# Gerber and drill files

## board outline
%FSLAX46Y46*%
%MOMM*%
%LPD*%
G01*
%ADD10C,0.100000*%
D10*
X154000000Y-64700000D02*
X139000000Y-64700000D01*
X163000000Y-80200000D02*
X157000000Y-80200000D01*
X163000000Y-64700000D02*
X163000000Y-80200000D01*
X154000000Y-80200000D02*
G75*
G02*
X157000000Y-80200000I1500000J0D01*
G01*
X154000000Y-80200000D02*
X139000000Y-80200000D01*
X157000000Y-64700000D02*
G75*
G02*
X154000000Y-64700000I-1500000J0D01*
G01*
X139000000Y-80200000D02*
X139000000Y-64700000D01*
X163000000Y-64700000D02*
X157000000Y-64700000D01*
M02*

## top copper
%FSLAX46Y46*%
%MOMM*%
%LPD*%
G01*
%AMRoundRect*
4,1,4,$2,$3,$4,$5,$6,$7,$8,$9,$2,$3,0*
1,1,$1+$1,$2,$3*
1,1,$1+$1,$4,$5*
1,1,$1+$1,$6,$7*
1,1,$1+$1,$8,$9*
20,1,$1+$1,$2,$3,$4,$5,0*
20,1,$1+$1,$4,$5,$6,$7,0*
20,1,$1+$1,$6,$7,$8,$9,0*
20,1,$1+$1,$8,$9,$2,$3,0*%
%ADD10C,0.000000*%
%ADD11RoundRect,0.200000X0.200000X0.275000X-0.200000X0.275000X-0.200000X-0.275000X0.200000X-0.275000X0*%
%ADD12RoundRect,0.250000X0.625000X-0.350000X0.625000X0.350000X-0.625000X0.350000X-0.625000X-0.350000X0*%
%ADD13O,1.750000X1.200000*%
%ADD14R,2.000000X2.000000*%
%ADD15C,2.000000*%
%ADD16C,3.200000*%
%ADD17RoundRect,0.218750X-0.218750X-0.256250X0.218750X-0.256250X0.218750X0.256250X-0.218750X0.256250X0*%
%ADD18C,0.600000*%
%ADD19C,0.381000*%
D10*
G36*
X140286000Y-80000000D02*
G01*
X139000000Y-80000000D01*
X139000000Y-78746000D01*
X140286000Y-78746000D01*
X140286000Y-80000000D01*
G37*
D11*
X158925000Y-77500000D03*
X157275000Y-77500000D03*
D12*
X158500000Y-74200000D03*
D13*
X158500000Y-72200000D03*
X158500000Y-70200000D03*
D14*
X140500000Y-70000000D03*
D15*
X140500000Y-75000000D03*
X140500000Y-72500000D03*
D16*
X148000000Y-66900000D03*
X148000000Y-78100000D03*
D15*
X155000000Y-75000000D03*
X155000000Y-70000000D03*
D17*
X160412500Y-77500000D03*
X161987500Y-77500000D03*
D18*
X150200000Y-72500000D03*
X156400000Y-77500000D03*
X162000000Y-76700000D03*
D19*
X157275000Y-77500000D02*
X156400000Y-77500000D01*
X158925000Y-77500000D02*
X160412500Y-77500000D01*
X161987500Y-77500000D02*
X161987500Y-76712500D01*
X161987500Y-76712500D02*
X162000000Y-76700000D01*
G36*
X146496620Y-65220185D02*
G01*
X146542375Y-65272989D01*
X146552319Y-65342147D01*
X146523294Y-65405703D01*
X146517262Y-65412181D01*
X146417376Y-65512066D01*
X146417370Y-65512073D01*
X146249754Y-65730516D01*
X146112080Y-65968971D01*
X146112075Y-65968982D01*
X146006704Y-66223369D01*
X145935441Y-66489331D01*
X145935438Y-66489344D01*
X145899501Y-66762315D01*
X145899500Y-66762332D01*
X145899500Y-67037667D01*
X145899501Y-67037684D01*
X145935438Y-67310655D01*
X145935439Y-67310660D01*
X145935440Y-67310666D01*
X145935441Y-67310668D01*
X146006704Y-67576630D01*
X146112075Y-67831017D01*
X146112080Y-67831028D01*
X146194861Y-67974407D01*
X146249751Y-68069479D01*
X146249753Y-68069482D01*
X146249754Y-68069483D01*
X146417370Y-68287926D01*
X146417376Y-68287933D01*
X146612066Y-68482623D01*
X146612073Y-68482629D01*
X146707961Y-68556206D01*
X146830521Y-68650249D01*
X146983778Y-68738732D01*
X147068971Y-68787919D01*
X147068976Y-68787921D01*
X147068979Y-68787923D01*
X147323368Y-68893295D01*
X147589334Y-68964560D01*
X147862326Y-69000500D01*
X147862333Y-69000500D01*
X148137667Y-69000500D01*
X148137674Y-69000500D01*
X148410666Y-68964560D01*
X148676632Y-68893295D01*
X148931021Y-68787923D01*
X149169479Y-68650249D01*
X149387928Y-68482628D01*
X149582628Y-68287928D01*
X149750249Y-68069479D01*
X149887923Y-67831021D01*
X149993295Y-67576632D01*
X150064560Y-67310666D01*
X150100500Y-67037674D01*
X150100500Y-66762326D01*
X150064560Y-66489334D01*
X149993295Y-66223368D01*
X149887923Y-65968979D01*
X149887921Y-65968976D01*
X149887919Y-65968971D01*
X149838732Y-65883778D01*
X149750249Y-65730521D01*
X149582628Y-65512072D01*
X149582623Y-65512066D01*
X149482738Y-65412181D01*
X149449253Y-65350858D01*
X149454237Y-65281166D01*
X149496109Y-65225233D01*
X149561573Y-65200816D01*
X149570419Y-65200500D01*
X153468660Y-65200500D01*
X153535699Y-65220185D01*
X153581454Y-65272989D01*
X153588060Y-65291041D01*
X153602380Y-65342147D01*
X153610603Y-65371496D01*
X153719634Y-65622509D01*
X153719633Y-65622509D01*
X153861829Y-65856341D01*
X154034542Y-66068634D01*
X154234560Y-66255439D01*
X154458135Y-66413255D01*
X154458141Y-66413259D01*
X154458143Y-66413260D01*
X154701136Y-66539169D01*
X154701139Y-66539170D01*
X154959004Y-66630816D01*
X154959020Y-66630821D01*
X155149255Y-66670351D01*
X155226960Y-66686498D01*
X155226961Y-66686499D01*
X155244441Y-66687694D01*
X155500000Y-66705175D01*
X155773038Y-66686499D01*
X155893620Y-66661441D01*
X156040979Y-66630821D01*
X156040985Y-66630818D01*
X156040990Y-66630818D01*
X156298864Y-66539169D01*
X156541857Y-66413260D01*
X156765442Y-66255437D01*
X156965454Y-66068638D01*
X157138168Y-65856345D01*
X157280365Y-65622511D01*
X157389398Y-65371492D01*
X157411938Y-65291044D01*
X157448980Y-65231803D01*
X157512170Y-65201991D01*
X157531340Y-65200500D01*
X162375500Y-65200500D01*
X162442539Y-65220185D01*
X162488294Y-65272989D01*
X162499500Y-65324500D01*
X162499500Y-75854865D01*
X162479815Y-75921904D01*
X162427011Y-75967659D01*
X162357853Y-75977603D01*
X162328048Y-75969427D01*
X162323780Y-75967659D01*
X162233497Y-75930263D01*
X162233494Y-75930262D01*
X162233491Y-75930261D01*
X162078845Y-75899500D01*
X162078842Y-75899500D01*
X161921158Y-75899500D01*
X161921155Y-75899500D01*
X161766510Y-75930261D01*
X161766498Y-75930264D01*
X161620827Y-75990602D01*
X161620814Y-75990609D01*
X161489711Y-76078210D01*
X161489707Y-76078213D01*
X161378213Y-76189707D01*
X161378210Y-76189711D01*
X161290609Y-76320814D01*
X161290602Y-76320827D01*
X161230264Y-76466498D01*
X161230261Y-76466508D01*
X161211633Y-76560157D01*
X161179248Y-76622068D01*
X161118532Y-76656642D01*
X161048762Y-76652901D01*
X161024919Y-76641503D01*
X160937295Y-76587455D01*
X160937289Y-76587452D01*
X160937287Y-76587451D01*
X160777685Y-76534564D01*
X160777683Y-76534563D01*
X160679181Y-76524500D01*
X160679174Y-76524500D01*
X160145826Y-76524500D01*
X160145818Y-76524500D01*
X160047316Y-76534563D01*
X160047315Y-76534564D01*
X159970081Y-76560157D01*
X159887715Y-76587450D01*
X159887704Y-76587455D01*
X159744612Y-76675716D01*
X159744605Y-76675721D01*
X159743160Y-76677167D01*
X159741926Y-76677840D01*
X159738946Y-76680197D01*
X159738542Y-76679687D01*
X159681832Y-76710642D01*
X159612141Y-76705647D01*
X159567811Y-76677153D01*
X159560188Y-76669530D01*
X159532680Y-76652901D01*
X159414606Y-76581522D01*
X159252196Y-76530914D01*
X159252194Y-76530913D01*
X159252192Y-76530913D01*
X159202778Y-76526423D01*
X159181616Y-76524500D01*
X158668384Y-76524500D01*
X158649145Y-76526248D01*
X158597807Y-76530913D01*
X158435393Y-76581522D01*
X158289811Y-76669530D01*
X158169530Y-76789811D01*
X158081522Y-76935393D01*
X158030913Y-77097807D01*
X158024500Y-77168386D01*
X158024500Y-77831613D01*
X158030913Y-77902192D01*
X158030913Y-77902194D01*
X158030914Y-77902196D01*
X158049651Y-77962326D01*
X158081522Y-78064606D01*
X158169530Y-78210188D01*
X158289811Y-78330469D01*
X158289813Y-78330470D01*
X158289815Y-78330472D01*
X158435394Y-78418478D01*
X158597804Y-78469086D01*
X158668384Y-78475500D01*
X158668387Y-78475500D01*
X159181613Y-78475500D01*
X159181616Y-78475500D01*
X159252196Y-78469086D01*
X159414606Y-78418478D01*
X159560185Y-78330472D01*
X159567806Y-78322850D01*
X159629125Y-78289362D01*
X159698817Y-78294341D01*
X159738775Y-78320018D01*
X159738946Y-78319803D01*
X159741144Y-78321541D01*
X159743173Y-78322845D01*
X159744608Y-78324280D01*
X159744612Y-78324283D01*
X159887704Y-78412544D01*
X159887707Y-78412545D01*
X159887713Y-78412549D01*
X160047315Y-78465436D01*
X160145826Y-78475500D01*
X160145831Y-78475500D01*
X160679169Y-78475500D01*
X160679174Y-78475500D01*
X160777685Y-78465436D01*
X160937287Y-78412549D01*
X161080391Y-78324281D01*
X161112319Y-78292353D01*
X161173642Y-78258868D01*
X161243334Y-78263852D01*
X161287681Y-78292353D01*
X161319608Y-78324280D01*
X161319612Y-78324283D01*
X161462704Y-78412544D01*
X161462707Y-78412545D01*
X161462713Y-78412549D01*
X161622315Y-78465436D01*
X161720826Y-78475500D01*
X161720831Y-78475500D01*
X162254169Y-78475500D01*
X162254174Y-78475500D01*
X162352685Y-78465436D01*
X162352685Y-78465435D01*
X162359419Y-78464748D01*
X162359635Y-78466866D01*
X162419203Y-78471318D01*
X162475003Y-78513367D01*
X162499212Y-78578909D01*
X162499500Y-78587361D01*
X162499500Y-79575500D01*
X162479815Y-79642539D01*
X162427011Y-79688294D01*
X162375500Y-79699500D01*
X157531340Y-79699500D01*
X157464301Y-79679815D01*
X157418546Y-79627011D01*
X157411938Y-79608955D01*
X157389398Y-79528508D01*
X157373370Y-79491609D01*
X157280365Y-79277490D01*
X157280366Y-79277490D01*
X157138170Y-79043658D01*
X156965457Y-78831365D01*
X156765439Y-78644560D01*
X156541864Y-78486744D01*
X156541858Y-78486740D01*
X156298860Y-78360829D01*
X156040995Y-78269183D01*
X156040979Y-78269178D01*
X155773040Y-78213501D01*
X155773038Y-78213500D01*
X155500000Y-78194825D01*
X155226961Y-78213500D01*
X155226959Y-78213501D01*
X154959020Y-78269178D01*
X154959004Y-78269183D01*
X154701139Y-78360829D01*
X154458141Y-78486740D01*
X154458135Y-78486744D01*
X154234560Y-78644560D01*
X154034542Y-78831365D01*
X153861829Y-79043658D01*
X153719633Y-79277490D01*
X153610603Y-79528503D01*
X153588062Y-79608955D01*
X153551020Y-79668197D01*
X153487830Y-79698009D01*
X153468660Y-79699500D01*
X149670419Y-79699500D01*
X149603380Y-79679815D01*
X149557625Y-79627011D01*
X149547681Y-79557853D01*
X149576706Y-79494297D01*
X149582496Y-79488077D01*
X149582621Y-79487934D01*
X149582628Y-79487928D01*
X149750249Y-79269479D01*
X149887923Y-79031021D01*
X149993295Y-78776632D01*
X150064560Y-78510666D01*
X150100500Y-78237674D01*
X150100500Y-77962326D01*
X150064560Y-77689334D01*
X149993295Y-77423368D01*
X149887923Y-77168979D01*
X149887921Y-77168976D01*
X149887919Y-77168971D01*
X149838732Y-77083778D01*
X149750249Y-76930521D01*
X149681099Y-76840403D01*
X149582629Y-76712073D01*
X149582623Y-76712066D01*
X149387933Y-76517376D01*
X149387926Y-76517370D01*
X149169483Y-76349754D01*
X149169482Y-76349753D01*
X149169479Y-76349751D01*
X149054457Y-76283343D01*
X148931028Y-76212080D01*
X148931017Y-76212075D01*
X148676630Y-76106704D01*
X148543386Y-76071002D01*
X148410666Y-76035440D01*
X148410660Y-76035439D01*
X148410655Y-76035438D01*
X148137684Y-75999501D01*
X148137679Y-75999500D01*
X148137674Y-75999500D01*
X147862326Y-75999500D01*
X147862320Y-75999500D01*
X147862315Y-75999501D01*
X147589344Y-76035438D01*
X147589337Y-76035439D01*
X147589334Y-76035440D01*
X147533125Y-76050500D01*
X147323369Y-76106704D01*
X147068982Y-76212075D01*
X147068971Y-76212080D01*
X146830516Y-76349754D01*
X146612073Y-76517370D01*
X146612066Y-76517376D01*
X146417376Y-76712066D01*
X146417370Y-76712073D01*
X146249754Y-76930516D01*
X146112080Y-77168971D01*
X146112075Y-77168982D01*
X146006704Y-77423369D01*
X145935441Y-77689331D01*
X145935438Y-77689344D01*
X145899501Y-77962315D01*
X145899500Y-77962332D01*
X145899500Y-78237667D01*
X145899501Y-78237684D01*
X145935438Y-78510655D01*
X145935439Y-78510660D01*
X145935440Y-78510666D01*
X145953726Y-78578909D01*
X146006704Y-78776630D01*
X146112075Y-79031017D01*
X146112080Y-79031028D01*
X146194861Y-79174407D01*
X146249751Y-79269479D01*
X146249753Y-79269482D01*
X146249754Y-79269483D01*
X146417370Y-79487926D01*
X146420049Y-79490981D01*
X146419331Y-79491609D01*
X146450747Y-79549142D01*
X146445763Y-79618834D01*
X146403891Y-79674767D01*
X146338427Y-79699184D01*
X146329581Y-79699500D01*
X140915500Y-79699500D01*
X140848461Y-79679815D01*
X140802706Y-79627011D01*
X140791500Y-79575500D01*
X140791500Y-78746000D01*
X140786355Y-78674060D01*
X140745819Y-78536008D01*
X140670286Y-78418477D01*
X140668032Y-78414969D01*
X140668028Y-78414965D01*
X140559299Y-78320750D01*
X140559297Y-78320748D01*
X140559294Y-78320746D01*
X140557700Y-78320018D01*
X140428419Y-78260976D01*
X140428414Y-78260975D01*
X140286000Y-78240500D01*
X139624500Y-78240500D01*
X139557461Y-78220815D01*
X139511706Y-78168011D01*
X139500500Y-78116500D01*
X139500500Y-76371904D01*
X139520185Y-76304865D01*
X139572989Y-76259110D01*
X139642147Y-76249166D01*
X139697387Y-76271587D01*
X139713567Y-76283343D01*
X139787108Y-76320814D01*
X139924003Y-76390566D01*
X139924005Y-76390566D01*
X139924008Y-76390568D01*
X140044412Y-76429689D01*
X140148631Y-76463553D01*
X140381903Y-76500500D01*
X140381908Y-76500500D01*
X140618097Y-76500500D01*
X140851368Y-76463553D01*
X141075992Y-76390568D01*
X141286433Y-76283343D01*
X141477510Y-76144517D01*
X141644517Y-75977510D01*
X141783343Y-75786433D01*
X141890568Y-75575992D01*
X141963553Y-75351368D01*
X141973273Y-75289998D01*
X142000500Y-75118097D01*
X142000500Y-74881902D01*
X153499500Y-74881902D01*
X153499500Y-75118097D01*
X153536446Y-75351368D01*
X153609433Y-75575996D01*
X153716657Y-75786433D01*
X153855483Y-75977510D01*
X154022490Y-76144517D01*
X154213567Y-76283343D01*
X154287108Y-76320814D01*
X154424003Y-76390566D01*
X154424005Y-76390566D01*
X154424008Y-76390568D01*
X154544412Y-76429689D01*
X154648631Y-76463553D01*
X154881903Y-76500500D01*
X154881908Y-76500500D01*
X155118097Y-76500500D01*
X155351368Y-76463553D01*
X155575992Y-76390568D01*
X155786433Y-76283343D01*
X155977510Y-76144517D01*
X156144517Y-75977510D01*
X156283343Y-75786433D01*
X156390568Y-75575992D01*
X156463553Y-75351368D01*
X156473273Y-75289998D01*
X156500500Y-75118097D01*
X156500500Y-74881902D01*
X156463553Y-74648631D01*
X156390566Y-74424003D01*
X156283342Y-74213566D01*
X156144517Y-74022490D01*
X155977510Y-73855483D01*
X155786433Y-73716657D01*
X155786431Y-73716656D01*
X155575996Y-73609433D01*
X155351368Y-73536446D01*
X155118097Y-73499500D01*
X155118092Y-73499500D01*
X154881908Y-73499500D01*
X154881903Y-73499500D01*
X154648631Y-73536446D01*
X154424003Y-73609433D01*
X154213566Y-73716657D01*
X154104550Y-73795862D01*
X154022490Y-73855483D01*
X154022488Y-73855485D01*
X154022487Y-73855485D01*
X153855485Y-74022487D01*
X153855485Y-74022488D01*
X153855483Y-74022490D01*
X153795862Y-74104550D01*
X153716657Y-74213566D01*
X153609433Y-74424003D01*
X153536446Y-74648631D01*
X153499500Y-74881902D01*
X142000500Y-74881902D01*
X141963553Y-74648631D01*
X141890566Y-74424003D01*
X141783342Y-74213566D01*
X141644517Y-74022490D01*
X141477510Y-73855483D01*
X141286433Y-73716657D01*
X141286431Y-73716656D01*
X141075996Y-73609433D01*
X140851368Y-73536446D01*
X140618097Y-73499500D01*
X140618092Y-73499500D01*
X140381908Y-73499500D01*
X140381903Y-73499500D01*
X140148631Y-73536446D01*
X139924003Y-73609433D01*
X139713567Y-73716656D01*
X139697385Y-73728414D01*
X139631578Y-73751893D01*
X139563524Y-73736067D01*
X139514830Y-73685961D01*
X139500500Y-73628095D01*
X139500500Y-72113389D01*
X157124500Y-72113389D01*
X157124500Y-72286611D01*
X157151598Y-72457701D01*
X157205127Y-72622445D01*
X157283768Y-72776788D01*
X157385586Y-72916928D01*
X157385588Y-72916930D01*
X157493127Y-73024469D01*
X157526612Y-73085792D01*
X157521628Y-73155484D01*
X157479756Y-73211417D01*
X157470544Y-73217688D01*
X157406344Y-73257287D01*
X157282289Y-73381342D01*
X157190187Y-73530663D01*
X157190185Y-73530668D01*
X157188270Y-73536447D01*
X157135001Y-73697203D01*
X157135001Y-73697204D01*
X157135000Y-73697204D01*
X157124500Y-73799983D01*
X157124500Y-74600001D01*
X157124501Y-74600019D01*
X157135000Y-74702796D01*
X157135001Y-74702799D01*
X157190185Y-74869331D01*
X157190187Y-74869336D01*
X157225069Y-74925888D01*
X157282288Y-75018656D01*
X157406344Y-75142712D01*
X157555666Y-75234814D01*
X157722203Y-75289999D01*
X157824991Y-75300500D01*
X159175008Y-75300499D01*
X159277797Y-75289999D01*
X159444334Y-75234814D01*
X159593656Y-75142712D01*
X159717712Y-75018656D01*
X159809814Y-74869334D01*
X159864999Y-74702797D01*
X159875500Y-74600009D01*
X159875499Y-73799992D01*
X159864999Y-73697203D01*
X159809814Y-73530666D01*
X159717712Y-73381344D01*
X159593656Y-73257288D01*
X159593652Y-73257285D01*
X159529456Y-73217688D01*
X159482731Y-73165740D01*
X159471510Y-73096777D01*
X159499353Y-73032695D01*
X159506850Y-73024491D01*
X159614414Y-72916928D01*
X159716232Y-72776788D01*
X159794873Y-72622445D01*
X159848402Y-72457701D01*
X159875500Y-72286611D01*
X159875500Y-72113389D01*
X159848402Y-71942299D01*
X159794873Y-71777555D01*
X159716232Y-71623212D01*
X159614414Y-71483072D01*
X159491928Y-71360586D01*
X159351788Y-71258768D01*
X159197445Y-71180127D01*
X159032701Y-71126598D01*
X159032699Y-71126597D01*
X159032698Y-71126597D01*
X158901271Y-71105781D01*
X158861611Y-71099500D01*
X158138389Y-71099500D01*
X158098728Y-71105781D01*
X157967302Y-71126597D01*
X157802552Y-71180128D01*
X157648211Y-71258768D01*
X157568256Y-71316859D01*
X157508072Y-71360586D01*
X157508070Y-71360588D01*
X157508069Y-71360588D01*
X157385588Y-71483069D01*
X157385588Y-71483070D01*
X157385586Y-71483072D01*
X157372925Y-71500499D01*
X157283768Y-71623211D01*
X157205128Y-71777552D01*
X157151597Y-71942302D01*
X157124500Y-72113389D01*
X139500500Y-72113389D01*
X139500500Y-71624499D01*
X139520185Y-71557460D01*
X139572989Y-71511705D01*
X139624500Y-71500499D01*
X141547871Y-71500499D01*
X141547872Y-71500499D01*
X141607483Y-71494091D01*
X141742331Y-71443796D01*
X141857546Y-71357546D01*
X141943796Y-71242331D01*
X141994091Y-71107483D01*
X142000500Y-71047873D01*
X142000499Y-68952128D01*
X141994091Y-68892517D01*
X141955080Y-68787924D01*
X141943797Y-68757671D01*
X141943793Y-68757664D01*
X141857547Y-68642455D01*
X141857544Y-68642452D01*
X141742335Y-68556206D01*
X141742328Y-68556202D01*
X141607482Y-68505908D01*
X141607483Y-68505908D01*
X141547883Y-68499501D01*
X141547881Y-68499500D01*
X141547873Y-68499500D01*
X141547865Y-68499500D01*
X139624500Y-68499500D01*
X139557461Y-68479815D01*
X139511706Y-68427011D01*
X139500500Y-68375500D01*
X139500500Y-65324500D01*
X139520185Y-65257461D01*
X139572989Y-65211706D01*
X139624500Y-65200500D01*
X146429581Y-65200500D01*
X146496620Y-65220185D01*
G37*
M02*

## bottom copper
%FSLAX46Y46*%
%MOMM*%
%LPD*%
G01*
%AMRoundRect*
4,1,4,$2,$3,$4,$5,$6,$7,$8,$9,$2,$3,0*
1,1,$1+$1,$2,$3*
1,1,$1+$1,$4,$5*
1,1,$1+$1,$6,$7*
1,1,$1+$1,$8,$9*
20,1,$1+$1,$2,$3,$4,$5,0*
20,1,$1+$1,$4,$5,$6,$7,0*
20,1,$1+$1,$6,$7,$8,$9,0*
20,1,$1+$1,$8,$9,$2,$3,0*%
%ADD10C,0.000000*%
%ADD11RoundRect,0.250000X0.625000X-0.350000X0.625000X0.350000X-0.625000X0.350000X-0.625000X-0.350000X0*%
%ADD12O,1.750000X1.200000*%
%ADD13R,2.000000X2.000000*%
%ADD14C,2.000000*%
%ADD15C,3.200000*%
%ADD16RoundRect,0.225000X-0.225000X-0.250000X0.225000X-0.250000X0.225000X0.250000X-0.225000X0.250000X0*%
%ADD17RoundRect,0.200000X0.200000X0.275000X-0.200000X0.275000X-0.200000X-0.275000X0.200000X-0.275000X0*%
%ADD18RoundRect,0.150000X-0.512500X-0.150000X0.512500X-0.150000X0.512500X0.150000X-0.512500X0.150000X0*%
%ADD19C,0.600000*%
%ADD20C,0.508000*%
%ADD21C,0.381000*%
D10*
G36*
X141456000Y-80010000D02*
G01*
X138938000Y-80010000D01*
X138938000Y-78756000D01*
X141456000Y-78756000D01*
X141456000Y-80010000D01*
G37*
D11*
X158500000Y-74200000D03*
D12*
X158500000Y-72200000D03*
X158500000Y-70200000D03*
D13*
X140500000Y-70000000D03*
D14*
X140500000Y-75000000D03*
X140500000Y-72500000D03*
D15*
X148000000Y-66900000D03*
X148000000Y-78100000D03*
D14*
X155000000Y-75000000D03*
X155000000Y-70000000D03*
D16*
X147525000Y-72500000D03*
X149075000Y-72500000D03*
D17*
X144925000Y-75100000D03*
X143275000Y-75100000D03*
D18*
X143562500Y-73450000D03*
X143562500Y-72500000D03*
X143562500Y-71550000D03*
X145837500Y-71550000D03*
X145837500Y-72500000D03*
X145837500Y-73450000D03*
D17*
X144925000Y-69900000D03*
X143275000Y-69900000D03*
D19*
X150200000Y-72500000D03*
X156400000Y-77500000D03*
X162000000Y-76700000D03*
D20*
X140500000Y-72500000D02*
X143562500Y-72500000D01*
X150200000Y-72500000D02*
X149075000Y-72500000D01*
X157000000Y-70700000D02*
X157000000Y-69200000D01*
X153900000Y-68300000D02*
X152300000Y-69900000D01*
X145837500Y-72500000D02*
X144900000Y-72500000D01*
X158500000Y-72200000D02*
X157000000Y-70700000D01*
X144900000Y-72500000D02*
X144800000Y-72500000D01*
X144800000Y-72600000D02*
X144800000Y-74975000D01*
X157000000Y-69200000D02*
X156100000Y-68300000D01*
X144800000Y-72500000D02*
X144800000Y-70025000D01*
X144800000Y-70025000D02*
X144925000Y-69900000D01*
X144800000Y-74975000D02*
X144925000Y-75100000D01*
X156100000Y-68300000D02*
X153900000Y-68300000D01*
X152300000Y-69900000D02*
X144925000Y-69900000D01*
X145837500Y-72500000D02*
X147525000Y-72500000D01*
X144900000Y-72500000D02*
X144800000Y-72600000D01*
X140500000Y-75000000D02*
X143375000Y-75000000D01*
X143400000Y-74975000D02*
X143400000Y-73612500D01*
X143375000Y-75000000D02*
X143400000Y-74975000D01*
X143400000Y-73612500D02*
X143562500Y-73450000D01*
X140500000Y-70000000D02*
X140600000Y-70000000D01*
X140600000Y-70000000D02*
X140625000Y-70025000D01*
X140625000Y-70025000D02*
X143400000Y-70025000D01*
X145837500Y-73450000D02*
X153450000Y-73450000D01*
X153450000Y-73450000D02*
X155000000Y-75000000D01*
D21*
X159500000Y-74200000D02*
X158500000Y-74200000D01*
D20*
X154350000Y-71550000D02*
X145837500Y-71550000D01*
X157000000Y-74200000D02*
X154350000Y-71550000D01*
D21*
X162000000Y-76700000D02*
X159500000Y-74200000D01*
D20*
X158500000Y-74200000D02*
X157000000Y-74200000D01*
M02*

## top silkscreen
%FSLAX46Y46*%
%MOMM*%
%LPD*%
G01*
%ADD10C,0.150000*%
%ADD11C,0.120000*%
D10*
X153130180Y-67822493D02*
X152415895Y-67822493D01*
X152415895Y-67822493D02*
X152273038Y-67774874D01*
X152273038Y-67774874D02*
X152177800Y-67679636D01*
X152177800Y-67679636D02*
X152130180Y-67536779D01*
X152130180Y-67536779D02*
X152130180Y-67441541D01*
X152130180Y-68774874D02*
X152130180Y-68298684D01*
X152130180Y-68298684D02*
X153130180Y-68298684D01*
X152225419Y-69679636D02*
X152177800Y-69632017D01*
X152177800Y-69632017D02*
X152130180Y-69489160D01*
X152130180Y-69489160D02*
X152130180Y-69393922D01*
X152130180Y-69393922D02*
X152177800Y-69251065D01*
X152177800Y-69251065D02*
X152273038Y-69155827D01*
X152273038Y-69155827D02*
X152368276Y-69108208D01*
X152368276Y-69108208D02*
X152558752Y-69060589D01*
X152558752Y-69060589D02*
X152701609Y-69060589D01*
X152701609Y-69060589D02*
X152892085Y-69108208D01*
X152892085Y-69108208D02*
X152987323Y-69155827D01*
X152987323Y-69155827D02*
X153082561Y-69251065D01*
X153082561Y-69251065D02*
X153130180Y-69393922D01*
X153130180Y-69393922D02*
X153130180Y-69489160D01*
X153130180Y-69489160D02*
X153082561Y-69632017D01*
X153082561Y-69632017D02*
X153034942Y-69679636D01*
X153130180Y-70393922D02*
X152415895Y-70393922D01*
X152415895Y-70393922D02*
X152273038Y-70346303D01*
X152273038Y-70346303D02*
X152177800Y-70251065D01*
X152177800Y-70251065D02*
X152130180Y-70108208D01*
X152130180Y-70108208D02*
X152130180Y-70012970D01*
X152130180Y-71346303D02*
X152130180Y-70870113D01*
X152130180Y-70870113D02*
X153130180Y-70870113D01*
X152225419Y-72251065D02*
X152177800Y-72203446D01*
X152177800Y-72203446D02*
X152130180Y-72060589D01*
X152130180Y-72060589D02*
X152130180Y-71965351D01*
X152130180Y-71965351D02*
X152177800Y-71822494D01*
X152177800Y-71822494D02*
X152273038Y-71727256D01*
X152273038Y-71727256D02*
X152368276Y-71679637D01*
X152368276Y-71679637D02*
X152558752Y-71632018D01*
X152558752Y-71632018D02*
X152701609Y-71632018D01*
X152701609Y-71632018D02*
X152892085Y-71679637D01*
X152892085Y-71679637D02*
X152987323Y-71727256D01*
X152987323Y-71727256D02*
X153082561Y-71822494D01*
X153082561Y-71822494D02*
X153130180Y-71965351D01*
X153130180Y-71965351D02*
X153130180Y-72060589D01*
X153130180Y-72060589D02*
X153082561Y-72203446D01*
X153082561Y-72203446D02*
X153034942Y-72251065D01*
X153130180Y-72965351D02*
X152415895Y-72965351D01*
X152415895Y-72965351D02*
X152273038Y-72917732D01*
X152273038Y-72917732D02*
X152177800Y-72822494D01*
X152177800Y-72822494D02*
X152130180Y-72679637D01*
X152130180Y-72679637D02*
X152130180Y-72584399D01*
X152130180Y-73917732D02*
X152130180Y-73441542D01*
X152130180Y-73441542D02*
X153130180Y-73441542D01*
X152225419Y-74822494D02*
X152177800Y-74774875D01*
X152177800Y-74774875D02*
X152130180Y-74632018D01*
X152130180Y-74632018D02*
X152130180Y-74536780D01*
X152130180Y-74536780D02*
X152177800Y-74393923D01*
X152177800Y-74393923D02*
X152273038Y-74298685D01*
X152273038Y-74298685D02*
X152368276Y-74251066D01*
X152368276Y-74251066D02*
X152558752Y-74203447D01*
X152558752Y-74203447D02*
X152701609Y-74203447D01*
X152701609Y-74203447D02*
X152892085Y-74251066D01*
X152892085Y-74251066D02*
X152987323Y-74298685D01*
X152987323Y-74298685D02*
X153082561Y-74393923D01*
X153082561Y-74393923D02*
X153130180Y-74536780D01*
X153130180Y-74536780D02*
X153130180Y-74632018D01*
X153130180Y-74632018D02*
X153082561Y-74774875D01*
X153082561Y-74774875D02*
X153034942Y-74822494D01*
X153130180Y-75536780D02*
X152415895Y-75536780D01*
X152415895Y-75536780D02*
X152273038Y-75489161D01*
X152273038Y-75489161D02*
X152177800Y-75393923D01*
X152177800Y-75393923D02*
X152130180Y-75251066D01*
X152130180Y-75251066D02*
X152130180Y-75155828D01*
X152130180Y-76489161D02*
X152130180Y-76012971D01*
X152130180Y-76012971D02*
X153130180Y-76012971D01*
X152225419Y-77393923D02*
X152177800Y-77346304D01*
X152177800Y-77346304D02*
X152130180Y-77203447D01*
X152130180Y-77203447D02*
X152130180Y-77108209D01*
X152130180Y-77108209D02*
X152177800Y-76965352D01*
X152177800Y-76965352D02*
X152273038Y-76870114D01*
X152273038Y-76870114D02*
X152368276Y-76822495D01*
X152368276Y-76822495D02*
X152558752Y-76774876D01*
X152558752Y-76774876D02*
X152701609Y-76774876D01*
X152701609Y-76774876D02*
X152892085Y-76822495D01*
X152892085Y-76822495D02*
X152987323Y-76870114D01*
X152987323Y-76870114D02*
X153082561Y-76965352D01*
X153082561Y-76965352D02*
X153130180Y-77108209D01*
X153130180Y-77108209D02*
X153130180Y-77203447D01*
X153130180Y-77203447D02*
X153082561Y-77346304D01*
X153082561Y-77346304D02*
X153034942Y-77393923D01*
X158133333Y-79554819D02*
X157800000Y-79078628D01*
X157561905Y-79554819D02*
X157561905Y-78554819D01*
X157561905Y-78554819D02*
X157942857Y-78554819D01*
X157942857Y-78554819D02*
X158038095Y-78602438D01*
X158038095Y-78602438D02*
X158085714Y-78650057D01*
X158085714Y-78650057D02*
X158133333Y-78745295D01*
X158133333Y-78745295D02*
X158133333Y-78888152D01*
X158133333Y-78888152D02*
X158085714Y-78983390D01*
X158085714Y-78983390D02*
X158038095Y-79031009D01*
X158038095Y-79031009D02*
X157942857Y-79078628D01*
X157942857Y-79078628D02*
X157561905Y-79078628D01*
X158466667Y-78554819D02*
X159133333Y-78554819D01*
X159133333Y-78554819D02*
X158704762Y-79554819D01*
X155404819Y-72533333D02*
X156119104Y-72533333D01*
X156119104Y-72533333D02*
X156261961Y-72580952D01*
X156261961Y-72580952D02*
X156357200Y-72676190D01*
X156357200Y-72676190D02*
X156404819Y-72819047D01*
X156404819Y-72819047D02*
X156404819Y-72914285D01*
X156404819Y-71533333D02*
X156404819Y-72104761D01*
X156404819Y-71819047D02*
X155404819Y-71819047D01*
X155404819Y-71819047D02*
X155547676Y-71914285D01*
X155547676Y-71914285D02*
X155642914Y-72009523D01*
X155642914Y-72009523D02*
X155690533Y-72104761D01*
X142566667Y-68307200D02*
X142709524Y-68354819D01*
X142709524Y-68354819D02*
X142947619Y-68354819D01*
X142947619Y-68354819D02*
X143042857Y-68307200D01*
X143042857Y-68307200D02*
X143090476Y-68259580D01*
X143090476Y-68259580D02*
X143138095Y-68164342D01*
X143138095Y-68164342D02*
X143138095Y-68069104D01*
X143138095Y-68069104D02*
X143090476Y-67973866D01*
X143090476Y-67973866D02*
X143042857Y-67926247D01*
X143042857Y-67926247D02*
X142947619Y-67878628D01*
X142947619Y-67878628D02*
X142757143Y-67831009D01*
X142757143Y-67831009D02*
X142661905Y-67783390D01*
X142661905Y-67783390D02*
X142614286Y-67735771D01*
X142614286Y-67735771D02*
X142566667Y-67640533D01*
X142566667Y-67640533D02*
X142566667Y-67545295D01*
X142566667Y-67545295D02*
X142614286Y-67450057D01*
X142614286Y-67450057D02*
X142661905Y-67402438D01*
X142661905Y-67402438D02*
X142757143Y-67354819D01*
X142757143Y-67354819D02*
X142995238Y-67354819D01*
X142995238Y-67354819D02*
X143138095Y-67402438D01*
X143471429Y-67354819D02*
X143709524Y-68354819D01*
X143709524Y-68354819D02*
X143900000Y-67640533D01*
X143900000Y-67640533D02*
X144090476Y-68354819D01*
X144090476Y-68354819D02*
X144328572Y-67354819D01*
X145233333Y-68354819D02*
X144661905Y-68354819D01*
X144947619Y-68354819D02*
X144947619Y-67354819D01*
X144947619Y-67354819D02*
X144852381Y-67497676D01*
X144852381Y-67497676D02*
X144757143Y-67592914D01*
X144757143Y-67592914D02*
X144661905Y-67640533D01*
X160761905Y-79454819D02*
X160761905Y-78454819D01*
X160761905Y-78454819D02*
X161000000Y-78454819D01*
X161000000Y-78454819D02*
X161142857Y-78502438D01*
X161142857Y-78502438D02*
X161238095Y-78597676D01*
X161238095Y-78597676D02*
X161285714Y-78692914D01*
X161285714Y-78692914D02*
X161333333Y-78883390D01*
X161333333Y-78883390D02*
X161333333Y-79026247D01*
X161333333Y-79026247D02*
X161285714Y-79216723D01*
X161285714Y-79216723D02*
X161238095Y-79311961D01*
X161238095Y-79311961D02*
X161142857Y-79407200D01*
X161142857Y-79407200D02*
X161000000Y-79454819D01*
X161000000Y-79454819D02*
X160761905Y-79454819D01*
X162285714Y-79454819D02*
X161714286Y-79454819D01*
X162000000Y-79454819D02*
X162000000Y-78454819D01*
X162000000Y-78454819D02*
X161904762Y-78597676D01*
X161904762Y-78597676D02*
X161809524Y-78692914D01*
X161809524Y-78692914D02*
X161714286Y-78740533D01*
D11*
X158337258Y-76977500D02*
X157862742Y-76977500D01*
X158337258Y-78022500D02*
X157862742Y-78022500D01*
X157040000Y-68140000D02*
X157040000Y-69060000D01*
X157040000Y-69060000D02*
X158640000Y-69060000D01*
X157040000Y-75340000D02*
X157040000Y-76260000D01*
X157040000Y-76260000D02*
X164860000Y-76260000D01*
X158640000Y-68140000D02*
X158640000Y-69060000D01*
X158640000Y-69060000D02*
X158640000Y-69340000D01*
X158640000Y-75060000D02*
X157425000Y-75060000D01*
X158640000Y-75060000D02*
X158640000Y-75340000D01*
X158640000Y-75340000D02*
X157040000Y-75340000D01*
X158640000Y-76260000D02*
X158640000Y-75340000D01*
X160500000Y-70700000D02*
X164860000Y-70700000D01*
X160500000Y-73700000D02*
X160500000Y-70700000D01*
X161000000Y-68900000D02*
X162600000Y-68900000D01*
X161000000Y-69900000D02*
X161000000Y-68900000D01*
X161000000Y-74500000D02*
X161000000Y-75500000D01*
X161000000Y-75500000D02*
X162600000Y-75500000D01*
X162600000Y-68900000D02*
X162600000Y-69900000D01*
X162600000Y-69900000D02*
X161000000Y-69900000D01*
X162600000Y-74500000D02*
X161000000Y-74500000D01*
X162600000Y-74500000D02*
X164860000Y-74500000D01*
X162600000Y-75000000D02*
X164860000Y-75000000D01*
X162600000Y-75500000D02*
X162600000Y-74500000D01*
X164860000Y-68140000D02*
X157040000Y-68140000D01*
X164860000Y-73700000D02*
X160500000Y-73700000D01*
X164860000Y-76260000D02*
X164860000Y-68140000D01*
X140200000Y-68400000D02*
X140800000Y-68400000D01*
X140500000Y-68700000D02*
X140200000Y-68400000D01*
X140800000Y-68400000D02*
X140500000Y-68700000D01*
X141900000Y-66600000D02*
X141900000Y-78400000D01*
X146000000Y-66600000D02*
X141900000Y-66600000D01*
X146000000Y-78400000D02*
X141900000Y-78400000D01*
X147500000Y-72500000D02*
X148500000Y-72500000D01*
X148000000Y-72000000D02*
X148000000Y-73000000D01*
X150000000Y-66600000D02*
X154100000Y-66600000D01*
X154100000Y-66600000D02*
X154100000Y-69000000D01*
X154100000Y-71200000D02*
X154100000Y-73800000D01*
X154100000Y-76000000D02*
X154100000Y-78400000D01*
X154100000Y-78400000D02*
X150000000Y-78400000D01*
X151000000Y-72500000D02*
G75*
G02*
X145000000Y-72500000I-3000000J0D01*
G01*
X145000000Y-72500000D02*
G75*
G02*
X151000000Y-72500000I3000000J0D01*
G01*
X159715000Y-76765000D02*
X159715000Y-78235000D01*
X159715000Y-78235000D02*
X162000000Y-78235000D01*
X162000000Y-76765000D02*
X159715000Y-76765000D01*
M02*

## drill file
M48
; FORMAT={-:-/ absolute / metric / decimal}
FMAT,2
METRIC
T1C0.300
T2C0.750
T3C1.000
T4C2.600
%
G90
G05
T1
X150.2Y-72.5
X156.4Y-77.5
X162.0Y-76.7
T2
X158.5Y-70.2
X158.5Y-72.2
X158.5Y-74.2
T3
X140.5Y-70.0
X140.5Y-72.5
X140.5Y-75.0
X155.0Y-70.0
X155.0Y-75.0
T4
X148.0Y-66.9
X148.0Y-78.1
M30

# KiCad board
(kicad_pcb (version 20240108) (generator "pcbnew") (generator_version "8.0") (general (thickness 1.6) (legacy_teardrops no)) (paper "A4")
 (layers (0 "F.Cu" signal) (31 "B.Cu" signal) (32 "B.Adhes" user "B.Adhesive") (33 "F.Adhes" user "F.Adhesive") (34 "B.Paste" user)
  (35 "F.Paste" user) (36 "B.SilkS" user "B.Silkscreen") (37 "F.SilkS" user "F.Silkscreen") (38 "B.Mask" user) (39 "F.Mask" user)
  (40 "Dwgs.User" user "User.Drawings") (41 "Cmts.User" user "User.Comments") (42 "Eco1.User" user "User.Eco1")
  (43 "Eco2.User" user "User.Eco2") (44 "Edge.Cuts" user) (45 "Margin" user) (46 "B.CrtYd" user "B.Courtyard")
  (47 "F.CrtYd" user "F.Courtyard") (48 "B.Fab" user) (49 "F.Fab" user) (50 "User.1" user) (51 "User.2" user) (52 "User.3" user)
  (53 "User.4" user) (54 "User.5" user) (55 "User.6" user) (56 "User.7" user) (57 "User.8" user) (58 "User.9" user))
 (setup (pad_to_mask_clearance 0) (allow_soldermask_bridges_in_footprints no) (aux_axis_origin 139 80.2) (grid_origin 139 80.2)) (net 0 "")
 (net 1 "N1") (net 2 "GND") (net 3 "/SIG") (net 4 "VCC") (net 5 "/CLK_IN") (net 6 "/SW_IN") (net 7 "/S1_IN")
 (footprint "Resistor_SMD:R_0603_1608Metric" (layer "F.Cu") (at 158.1 77.5 180)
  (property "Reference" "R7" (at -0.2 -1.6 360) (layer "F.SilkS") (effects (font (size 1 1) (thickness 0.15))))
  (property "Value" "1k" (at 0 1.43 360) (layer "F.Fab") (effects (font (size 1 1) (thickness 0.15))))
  (fp_line (start -0.237258 0.5225) (end 0.237258 0.5225) (stroke (width 0.12) (type solid)) (layer "F.SilkS"))
  (fp_line (start -0.237258 -0.5225) (end 0.237258 -0.5225) (stroke (width 0.12) (type solid)) (layer "F.SilkS"))
  (pad "1" smd roundrect (at -0.825 0 180) (size 0.8 0.95) (layers "F.Cu" "F.Paste" "F.Mask") (roundrect_rratio 0.25) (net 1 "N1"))
  (pad "2" smd roundrect (at 0.825 0 180) (size 0.8 0.95) (layers "F.Cu" "F.Paste" "F.Mask") (roundrect_rratio 0.25) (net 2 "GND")))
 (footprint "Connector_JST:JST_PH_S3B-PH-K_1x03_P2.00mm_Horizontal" (layer "F.Cu") (at 158.5 74.2 90)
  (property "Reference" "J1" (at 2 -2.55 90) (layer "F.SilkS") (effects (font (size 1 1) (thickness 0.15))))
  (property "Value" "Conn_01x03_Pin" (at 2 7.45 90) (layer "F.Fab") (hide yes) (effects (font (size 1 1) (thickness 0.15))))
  (fp_line (start 6.06 -1.46) (end 5.14 -1.46) (stroke (width 0.12) (type solid)) (layer "F.SilkS"))
  (fp_line (start 5.14 -1.46) (end 5.14 0.14) (stroke (width 0.12) (type solid)) (layer "F.SilkS"))
  (fp_line (start -1.14 -1.46) (end -2.06 -1.46) (stroke (width 0.12) (type solid)) (layer "F.SilkS"))
  (fp_line (start -2.06 -1.46) (end -2.06 6.36) (stroke (width 0.12) (type solid)) (layer "F.SilkS"))
  (fp_line (start 6.06 0.14) (end 5.14 0.14) (stroke (width 0.12) (type solid)) (layer "F.SilkS"))
  (fp_line (start 5.14 0.14) (end 4.86 0.14) (stroke (width 0.12) (type solid)) (layer "F.SilkS"))
  (fp_line (start -0.86 0.14) (end -0.86 -1.075) (stroke (width 0.12) (type solid)) (layer "F.SilkS"))
  (fp_line (start -0.86 0.14) (end -1.14 0.14) (stroke (width 0.12) (type solid)) (layer "F.SilkS"))
  (fp_line (start -1.14 0.14) (end -1.14 -1.46) (stroke (width 0.12) (type solid)) (layer "F.SilkS"))
  (fp_line (start -2.06 0.14) (end -1.14 0.14) (stroke (width 0.12) (type solid)) (layer "F.SilkS"))
  (fp_line (start 3.5 2) (end 3.5 6.36) (stroke (width 0.12) (type solid)) (layer "F.SilkS"))
  (fp_line (start 0.5 2) (end 3.5 2) (stroke (width 0.12) (type solid)) (layer "F.SilkS"))
  (fp_line (start 5.3 2.5) (end 5.3 4.1) (stroke (width 0.12) (type solid)) (layer "F.SilkS"))
  (fp_line (start 4.3 2.5) (end 5.3 2.5) (stroke (width 0.12) (type solid)) (layer "F.SilkS"))
  (fp_line (start -0.3 2.5) (end -1.3 2.5) (stroke (width 0.12) (type solid)) (layer "F.SilkS"))
  (fp_line (start -1.3 2.5) (end -1.3 4.1) (stroke (width 0.12) (type solid)) (layer "F.SilkS"))
  (fp_line (start 5.3 4.1) (end 4.3 4.1) (stroke (width 0.12) (type solid)) (layer "F.SilkS"))
  (fp_line (start 4.3 4.1) (end 4.3 2.5) (stroke (width 0.12) (type solid)) (layer "F.SilkS"))
  (fp_line (start -0.3 4.1) (end -0.3 2.5) (stroke (width 0.12) (type solid)) (layer "F.SilkS"))
  (fp_line (start -0.3 4.1) (end -0.3 6.36) (stroke (width 0.12) (type solid)) (layer "F.SilkS"))
  (fp_line (start -0.8 4.1) (end -0.8 6.36) (stroke (width 0.12) (type solid)) (layer "F.SilkS"))
  (fp_line (start -1.3 4.1) (end -0.3 4.1) (stroke (width 0.12) (type solid)) (layer "F.SilkS"))
  (fp_line (start 6.06 6.36) (end 6.06 -1.46) (stroke (width 0.12) (type solid)) (layer "F.SilkS"))
  (fp_line (start 0.5 6.36) (end 0.5 2) (stroke (width 0.12) (type solid)) (layer "F.SilkS"))
  (fp_line (start -2.06 6.36) (end 6.06 6.36) (stroke (width 0.12) (type solid)) (layer "F.SilkS"))
  (pad "1" thru_hole roundrect (at 0 0 90) (size 1.2 1.75) (drill 0.75) (layers "*.Cu" "*.Mask") (remove_unused_layers no)
   (roundrect_rratio 0.208333) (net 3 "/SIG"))
  (pad "2" thru_hole oval (at 2 0 90) (size 1.2 1.75) (drill 0.75) (layers "*.Cu" "*.Mask") (remove_unused_layers no) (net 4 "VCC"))
  (pad "3" thru_hole oval (at 4 0 90) (size 1.2 1.75) (drill 0.75) (layers "*.Cu" "*.Mask") (remove_unused_layers no) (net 2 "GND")))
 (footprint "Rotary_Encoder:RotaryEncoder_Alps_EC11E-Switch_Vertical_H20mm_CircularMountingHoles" (layer "F.Cu") (at 140.5 70)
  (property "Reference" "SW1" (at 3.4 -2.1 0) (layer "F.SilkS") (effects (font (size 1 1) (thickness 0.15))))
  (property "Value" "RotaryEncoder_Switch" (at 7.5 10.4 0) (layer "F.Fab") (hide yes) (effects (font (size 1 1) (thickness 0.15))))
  (fp_line (start -0.3 -1.6) (end 0.3 -1.6) (stroke (width 0.12) (type solid)) (layer "F.SilkS"))
  (fp_line (start 0 -1.3) (end -0.3 -1.6) (stroke (width 0.12) (type solid)) (layer "F.SilkS"))
  (fp_line (start 0.3 -1.6) (end 0 -1.3) (stroke (width 0.12) (type solid)) (layer "F.SilkS"))
  (fp_line (start 1.4 -3.4) (end 1.4 8.4) (stroke (width 0.12) (type solid)) (layer "F.SilkS"))
  (fp_line (start 5.5 -3.4) (end 1.4 -3.4) (stroke (width 0.12) (type solid)) (layer "F.SilkS"))
  (fp_line (start 5.5 8.4) (end 1.4 8.4) (stroke (width 0.12) (type solid)) (layer "F.SilkS"))
  (fp_line (start 7 2.5) (end 8 2.5) (stroke (width 0.12) (type solid)) (layer "F.SilkS"))
  (fp_line (start 7.5 2) (end 7.5 3) (stroke (width 0.12) (type solid)) (layer "F.SilkS"))
  (fp_line (start 9.5 -3.4) (end 13.6 -3.4) (stroke (width 0.12) (type solid)) (layer "F.SilkS"))
  (fp_line (start 13.6 -3.4) (end 13.6 -1) (stroke (width 0.12) (type solid)) (layer "F.SilkS"))
  (fp_line (start 13.6 1.2) (end 13.6 3.8) (stroke (width 0.12) (type solid)) (layer "F.SilkS"))
  (fp_line (start 13.6 6) (end 13.6 8.4) (stroke (width 0.12) (type solid)) (layer "F.SilkS"))
  (fp_line (start 13.6 8.4) (end 9.5 8.4) (stroke (width 0.12) (type solid)) (layer "F.SilkS"))
  (fp_circle (center 7.5 2.5) (end 10.5 2.5) (stroke (width 0.12) (type solid)) (fill none) (layer "F.SilkS"))
  (pad "A" thru_hole rect (at 0 0) (size 2 2) (drill 1) (layers "*.Cu" "*.Mask") (remove_unused_layers no) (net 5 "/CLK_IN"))
  (pad "B" thru_hole circle (at 0 5) (size 2 2) (drill 1) (layers "*.Cu" "*.Mask") (remove_unused_layers no) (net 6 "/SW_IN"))
  (pad "C" thru_hole circle (at 0 2.5) (size 2 2) (drill 1) (layers "*.Cu" "*.Mask") (remove_unused_layers no) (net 2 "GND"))
  (pad "MP" thru_hole circle (at 7.5 -3.1) (size 3.2 3.2) (drill 2.6) (layers "*.Cu" "*.Mask") (remove_unused_layers no))
  (pad "MP" thru_hole circle (at 7.5 8.1) (size 3.2 3.2) (drill 2.6) (layers "*.Cu" "*.Mask") (remove_unused_layers no))
  (pad "S1" thru_hole circle (at 14.5 5) (size 2 2) (drill 1) (layers "*.Cu" "*.Mask") (remove_unused_layers no) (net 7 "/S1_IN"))
  (pad "S2" thru_hole circle (at 14.5 0) (size 2 2) (drill 1) (layers "*.Cu" "*.Mask") (remove_unused_layers no) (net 2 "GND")))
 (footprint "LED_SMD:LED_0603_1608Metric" (layer "F.Cu") (at 161.2 77.5)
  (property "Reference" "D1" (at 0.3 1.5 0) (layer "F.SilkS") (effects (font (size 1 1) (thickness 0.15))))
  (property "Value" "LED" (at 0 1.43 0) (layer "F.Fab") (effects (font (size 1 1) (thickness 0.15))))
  (fp_line (start -1.485 -0.735) (end -1.485 0.735) (stroke (width 0.12) (type solid)) (layer "F.SilkS"))
  (fp_line (start -1.485 0.735) (end 0.8 0.735) (stroke (width 0.12) (type solid)) (layer "F.SilkS"))
  (fp_line (start 0.8 -0.735) (end -1.485 -0.735) (stroke (width 0.12) (type solid)) (layer "F.SilkS"))
  (pad "1" smd roundrect (at -0.7875 0) (size 0.875 0.95) (layers "F.Cu" "F.Paste" "F.Mask") (roundrect_rratio 0.25) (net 1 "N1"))
  (pad "2" smd roundrect (at 0.7875 0) (size 0.875 0.95) (layers "F.Cu" "F.Paste" "F.Mask") (roundrect_rratio 0.25) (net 3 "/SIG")))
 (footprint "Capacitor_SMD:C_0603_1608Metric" (layer "B.Cu") (at 148.3 72.5)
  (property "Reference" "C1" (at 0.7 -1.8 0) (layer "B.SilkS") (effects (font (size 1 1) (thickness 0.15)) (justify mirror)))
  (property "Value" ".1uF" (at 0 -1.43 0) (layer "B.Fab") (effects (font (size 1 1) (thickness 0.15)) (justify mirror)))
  (pad "1" smd roundrect (at -0.775 0) (size 0.9 0.95) (layers "B.Cu" "B.Paste" "B.Mask") (roundrect_rratio 0.25) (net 4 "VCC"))
  (pad "2" smd roundrect (at 0.775 0) (size 0.9 0.95) (layers "B.Cu" "B.Paste" "B.Mask") (roundrect_rratio 0.25) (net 2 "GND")))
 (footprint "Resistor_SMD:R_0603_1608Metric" (layer "B.Cu") (at 144.1 75.1 180)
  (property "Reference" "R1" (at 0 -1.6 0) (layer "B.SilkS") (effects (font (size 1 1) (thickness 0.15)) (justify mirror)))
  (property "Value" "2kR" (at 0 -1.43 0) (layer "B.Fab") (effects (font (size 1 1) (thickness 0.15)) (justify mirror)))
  (pad "1" smd roundrect (at -0.825 0 180) (size 0.8 0.95) (layers "B.Cu" "B.Paste" "B.Mask") (roundrect_rratio 0.25) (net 4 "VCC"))
  (pad "2" smd roundrect (at 0.825 0 180) (size 0.8 0.95) (layers "B.Cu" "B.Paste" "B.Mask") (roundrect_rratio 0.25) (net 6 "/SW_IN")))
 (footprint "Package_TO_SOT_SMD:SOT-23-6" (layer "B.Cu") (at 144.7 72.5)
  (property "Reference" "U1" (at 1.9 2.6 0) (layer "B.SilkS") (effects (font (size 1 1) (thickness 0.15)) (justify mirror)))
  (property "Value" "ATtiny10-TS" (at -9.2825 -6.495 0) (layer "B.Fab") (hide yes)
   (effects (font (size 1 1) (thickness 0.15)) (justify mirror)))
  (pad "1" smd roundrect (at -1.1375 0.95) (size 1.325 0.6) (layers "B.Cu" "B.Paste" "B.Mask") (roundrect_rratio 0.25) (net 6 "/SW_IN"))
  (pad "2" smd roundrect (at -1.1375 0) (size 1.325 0.6) (layers "B.Cu" "B.Paste" "B.Mask") (roundrect_rratio 0.25) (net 2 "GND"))
  (pad "3" smd roundrect (at -1.1375 -0.95) (size 1.325 0.6) (layers "B.Cu" "B.Paste" "B.Mask") (roundrect_rratio 0.25) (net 5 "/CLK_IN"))
  (pad "4" smd roundrect (at 1.1375 -0.95) (size 1.325 0.6) (layers "B.Cu" "B.Paste" "B.Mask") (roundrect_rratio 0.25) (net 3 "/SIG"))
  (pad "5" smd roundrect (at 1.1375 0) (size 1.325 0.6) (layers "B.Cu" "B.Paste" "B.Mask") (roundrect_rratio 0.25) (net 4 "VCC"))
  (pad "6" smd roundrect (at 1.1375 0.95) (size 1.325 0.6) (layers "B.Cu" "B.Paste" "B.Mask") (roundrect_rratio 0.25) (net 7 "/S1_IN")))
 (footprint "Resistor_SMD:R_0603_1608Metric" (layer "B.Cu") (at 144.1 69.9 180)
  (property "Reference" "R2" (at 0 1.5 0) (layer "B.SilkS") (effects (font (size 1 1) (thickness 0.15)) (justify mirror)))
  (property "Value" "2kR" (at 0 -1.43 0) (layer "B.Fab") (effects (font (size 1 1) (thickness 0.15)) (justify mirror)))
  (pad "1" smd roundrect (at -0.825 0 180) (size 0.8 0.95) (layers "B.Cu" "B.Paste" "B.Mask") (roundrect_rratio 0.25) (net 4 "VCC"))
  (pad "2" smd roundrect (at 0.825 0 180) (size 0.8 0.95) (layers "B.Cu" "B.Paste" "B.Mask") (roundrect_rratio 0.25) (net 5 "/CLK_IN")))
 (gr_poly (pts (xy 140.286 78.746) (xy 139 78.746) (xy 139 80) (xy 140.286 80)) (stroke (width 0) (type solid)) (fill solid) (layer "F.Cu"))
 (gr_poly
  (pts (xy 141.456 78.756) (xy 138.938 78.756) (xy 138.938 80.01) (xy 141.456 80.01)) (stroke (width 0) (type solid)) (fill solid)
  (layer "B.Cu"))
 (gr_line (start 154 64.7) (end 139 64.7) (stroke (width 0.1) (type default)) (layer "Edge.Cuts"))
 (gr_line (start 163 80.2) (end 157 80.2) (stroke (width 0.1) (type default)) (layer "Edge.Cuts"))
 (gr_line (start 163 64.7) (end 163 80.2) (stroke (width 0.1) (type default)) (layer "Edge.Cuts"))
 (gr_arc (start 154 80.2) (mid 155.5 78.7) (end 157 80.2) (stroke (width 0.1) (type default)) (layer "Edge.Cuts"))
 (gr_line (start 154 80.2) (end 139 80.2) (stroke (width 0.1) (type default)) (layer "Edge.Cuts"))
 (gr_arc (start 157 64.7) (mid 155.5 66.2) (end 154 64.7) (stroke (width 0.1) (type default)) (layer "Edge.Cuts"))
 (gr_line (start 139 80.2) (end 139 64.7) (stroke (width 0.1) (type default)) (layer "Edge.Cuts"))
 (gr_line (start 163 64.7) (end 157 64.7) (stroke (width 0.1) (type default)) (layer "Edge.Cuts"))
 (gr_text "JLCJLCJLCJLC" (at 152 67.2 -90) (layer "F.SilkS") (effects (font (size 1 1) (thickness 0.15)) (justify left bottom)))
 (segment (start 157.275 77.5) (end 156.4 77.5) (width 0.381) (layer "F.Cu") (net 2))
 (via (at 150.2 72.5) (size 0.6) (drill 0.3) (layers "F.Cu" "B.Cu") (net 2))
 (via (at 156.4 77.5) (size 0.6) (drill 0.3) (layers "F.Cu" "B.Cu") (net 2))
 (segment (start 140.5 72.5) (end 143.5625 72.5) (width 0.508) (layer "B.Cu") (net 2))
 (segment (start 150.2 72.5) (end 149.075 72.5) (width 0.508) (layer "B.Cu") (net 2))
 (segment (start 157 70.7) (end 157 69.2) (width 0.508) (layer "B.Cu") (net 4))
 (segment (start 153.9 68.3) (end 152.3 69.9) (width 0.508) (layer "B.Cu") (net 4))
 (segment (start 145.8375 72.5) (end 144.9 72.5) (width 0.508) (layer "B.Cu") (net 4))
 (segment (start 158.5 72.2) (end 157 70.7) (width 0.508) (layer "B.Cu") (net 4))
 (segment (start 144.9 72.5) (end 144.8 72.5) (width 0.508) (layer "B.Cu") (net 4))
 (segment (start 144.8 72.6) (end 144.8 74.975) (width 0.508) (layer "B.Cu") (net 4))
 (segment (start 157 69.2) (end 156.1 68.3) (width 0.508) (layer "B.Cu") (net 4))
 (segment (start 144.8 72.5) (end 144.8 70.025) (width 0.508) (layer "B.Cu") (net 4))
 (segment (start 144.8 70.025) (end 144.925 69.9) (width 0.508) (layer "B.Cu") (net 4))
 (segment (start 144.8 74.975) (end 144.925 75.1) (width 0.508) (layer "B.Cu") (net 4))
 (segment (start 156.1 68.3) (end 153.9 68.3) (width 0.508) (layer "B.Cu") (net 4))
 (segment (start 152.3 69.9) (end 144.925 69.9) (width 0.508) (layer "B.Cu") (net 4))
 (segment (start 145.8375 72.5) (end 147.525 72.5) (width 0.508) (layer "B.Cu") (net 4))
 (segment (start 144.9 72.5) (end 144.8 72.6) (width 0.508) (layer "B.Cu") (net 4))
 (segment (start 140.5 75) (end 143.375 75) (width 0.508) (layer "B.Cu") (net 6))
 (segment (start 143.4 74.975) (end 143.4 73.6125) (width 0.508) (layer "B.Cu") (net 6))
 (segment (start 143.375 75) (end 143.4 74.975) (width 0.508) (layer "B.Cu") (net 6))
 (segment (start 143.4 73.6125) (end 143.5625 73.45) (width 0.508) (layer "B.Cu") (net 6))
 (segment (start 140.5 70) (end 140.6 70) (width 0.508) (layer "B.Cu") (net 5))
 (segment (start 140.6 70) (end 140.625 70.025) (width 0.508) (layer "B.Cu") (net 5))
 (segment (start 140.625 70.025) (end 143.4 70.025) (width 0.508) (layer "B.Cu") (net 5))
 (segment (start 158.925 77.5) (end 160.4125 77.5) (width 0.381) (layer "F.Cu") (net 1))
 (segment (start 145.8375 73.45) (end 153.45 73.45) (width 0.508) (layer "B.Cu") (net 7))
 (segment (start 153.45 73.45) (end 155 75) (width 0.508) (layer "B.Cu") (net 7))
 (segment (start 161.9875 77.5) (end 161.9875 76.7125) (width 0.381) (layer "F.Cu") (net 3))
 (segment (start 161.9875 76.7125) (end 162 76.7) (width 0.381) (layer "F.Cu") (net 3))
 (via (at 162 76.7) (size 0.6) (drill 0.3) (layers "F.Cu" "B.Cu") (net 3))
 (segment (start 159.5 74.2) (end 158.5 74.2) (width 0.381) (layer "B.Cu") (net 3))
 (segment (start 154.35 71.55) (end 145.8375 71.55) (width 0.508) (layer "B.Cu") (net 3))
 (segment (start 157 74.2) (end 154.35 71.55) (width 0.508) (layer "B.Cu") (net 3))
 (segment (start 162 76.7) (end 159.5 74.2) (width 0.381) (layer "B.Cu") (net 3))
 (segment (start 158.5 74.2) (end 157 74.2) (width 0.508) (layer "B.Cu") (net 3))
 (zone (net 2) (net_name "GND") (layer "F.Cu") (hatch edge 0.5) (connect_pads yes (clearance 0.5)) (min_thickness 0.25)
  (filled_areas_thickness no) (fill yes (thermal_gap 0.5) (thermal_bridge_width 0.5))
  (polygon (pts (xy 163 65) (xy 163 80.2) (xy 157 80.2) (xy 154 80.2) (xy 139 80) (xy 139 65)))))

